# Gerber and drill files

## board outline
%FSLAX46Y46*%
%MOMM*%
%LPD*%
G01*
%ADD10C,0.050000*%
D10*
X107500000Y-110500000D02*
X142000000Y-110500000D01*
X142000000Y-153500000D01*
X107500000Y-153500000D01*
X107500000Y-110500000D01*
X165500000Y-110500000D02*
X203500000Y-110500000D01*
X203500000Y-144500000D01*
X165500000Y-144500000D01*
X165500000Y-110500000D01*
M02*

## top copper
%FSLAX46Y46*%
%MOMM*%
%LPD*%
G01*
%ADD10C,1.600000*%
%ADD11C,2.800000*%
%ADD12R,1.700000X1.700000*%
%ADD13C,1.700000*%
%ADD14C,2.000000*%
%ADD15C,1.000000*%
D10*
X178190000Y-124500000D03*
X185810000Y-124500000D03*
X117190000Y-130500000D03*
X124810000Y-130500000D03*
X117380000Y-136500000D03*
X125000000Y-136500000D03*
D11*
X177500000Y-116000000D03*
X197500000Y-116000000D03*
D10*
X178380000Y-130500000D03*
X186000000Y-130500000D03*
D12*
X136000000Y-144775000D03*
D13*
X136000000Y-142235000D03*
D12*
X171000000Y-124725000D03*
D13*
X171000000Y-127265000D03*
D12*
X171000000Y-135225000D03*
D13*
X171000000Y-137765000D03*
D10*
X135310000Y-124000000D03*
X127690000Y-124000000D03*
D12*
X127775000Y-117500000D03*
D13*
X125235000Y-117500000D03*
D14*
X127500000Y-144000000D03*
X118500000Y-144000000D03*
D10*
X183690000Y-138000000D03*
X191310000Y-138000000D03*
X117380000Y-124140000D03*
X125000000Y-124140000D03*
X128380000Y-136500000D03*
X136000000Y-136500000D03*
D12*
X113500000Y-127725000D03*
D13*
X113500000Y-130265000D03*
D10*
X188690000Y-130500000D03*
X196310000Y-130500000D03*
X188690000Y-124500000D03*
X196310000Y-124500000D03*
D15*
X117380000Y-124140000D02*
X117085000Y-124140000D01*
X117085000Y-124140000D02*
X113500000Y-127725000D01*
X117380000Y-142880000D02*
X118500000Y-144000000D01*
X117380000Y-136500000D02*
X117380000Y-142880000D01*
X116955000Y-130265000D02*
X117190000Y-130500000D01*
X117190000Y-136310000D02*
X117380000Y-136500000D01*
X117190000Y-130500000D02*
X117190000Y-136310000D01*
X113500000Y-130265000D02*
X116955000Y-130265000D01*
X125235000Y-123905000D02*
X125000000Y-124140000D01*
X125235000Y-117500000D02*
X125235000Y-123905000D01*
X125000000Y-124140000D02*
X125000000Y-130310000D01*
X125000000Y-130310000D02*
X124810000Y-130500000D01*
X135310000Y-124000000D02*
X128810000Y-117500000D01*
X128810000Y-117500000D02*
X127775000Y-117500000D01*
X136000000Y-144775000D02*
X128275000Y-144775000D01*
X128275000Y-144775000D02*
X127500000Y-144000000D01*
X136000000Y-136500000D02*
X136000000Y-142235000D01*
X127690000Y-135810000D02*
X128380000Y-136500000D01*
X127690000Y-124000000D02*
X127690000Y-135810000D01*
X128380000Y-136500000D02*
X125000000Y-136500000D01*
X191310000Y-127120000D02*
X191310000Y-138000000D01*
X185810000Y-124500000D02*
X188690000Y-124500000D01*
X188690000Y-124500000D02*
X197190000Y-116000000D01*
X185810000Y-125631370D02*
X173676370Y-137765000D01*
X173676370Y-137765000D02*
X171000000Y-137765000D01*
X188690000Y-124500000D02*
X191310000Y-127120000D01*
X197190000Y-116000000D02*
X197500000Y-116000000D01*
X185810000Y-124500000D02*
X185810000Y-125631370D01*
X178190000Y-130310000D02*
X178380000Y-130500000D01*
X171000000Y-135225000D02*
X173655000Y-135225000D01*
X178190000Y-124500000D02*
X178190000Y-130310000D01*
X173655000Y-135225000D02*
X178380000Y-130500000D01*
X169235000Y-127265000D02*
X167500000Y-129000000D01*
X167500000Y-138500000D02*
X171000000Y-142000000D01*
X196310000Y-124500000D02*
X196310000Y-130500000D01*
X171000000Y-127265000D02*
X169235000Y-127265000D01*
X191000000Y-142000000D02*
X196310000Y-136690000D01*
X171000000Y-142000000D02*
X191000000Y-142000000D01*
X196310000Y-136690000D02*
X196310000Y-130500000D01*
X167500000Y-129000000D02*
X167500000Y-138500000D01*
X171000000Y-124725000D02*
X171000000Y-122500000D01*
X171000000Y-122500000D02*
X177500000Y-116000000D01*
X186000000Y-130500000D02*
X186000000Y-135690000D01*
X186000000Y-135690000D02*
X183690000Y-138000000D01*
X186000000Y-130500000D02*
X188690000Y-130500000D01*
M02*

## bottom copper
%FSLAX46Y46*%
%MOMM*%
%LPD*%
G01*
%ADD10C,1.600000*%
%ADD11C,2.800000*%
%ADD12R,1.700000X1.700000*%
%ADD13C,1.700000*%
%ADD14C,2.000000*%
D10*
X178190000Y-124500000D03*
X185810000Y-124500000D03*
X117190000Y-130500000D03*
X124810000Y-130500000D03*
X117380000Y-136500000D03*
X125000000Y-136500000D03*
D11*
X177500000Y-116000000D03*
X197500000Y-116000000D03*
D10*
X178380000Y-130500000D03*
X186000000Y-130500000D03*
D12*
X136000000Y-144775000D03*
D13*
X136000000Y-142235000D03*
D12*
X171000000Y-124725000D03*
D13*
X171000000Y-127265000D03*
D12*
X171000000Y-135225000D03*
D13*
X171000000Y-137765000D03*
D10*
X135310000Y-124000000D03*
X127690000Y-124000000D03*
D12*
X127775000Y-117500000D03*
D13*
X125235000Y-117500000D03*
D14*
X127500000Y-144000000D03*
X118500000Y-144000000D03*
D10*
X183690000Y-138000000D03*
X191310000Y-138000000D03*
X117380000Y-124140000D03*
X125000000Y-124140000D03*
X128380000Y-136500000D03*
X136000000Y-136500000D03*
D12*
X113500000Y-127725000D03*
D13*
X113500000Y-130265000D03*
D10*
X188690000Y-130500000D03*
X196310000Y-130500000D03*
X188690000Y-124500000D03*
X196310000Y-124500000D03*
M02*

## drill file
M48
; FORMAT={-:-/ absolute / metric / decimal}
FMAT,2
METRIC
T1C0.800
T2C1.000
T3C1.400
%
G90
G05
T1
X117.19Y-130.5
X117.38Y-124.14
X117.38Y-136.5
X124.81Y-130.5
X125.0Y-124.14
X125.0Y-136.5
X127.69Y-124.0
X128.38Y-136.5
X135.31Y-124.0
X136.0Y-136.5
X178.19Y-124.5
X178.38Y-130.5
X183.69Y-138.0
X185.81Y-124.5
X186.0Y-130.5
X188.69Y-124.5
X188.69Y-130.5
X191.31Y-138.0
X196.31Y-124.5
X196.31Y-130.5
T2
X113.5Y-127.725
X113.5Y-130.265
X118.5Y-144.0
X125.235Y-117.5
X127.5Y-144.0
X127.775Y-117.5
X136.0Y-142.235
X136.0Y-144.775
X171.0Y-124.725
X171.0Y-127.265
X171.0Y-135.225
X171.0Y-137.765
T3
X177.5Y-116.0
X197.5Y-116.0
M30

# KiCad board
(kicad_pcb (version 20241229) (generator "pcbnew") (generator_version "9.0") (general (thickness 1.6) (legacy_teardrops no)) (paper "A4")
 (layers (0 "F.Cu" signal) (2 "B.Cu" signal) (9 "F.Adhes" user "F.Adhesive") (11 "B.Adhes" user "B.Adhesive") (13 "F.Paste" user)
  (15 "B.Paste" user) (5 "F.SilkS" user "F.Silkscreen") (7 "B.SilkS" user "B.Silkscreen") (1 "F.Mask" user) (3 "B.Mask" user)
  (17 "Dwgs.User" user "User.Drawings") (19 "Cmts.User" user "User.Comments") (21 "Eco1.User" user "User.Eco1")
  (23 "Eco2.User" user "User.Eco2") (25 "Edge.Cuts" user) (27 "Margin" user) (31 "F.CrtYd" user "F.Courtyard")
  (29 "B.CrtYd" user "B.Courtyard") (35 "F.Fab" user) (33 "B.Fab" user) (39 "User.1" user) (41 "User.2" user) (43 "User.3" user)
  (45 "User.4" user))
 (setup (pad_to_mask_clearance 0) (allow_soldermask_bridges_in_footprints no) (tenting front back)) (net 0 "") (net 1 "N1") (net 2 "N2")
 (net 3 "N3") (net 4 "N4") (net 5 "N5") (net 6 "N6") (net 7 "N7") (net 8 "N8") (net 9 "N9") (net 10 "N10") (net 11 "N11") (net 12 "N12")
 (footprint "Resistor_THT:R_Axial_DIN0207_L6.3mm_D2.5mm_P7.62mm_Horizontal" (layer "F.Cu") (at 178.19 124.5)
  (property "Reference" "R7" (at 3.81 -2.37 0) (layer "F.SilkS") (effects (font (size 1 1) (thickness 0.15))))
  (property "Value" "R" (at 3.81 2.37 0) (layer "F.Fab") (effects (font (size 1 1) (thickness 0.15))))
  (pad "1" thru_hole circle (at 0 0) (size 1.6 1.6) (drill 0.8) (layers "*.Cu" "*.Mask") (remove_unused_layers no) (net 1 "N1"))
  (pad "2" thru_hole circle (at 7.62 0) (size 1.6 1.6) (drill 0.8) (layers "*.Cu" "*.Mask") (remove_unused_layers no) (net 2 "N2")))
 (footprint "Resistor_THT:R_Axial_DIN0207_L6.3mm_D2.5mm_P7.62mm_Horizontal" (layer "F.Cu") (at 117.19 130.5)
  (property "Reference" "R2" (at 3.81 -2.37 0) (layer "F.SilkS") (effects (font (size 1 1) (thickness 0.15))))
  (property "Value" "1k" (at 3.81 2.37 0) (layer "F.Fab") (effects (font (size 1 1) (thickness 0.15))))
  (pad "1" thru_hole circle (at 0 0) (size 1.6 1.6) (drill 0.8) (layers "*.Cu" "*.Mask") (remove_unused_layers no) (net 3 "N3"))
  (pad "2" thru_hole circle (at 7.62 0) (size 1.6 1.6) (drill 0.8) (layers "*.Cu" "*.Mask") (remove_unused_layers no) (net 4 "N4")))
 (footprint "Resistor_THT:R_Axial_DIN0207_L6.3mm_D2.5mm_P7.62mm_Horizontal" (layer "F.Cu") (at 117.38 136.5)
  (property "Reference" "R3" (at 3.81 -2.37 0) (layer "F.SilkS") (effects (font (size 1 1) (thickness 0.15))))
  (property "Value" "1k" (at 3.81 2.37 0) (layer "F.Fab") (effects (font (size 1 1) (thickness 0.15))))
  (pad "1" thru_hole circle (at 0 0) (size 1.6 1.6) (drill 0.8) (layers "*.Cu" "*.Mask") (remove_unused_layers no) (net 3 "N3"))
  (pad "2" thru_hole circle (at 7.62 0) (size 1.6 1.6) (drill 0.8) (layers "*.Cu" "*.Mask") (remove_unused_layers no) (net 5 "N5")))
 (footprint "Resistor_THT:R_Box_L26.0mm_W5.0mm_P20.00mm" (layer "F.Cu") (at 177.5 116)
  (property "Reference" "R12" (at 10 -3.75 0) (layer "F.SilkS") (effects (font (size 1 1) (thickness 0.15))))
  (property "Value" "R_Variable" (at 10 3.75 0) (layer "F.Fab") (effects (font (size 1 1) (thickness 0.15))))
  (pad "1" thru_hole circle (at 0 0) (size 2.8 2.8) (drill 1.4) (layers "*.Cu" "*.Mask") (remove_unused_layers no) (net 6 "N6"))
  (pad "2" thru_hole circle (at 20 0) (size 2.8 2.8) (drill 1.4) (layers "*.Cu" "*.Mask") (remove_unused_layers no) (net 2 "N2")))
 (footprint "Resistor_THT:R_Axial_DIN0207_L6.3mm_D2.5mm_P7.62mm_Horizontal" (layer "F.Cu") (at 178.38 130.5)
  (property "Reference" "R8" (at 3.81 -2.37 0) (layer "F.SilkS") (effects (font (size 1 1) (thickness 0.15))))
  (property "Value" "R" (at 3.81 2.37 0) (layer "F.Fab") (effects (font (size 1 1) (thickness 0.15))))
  (pad "1" thru_hole circle (at 0 0) (size 1.6 1.6) (drill 0.8) (layers "*.Cu" "*.Mask") (remove_unused_layers no) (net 1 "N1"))
  (pad "2" thru_hole circle (at 7.62 0) (size 1.6 1.6) (drill 0.8) (layers "*.Cu" "*.Mask") (remove_unused_layers no) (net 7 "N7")))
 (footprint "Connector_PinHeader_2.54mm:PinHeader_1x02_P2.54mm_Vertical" (layer "F.Cu") (at 136 144.775 180)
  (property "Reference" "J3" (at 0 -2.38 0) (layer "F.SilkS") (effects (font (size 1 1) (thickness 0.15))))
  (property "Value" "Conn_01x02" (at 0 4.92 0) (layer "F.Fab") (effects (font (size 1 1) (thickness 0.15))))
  (pad "1" thru_hole rect (at 0 0 180) (size 1.7 1.7) (drill 1) (layers "*.Cu" "*.Mask") (remove_unused_layers no) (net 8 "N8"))
  (pad "2" thru_hole circle (at 0 2.54 180) (size 1.7 1.7) (drill 1) (layers "*.Cu" "*.Mask") (remove_unused_layers no) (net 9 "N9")))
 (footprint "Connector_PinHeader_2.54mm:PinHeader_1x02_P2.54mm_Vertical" (layer "F.Cu") (at 171 124.725)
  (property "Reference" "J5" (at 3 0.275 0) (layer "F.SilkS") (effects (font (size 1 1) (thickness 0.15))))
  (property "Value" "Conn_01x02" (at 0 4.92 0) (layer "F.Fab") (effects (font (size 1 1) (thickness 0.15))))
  (pad "1" thru_hole rect (at 0 0) (size 1.7 1.7) (drill 1) (layers "*.Cu" "*.Mask") (remove_unused_layers no) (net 6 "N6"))
  (pad "2" thru_hole circle (at 0 2.54) (size 1.7 1.7) (drill 1) (layers "*.Cu" "*.Mask") (remove_unused_layers no) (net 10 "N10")))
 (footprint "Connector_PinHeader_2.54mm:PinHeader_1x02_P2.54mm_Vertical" (layer "F.Cu") (at 171 135.225)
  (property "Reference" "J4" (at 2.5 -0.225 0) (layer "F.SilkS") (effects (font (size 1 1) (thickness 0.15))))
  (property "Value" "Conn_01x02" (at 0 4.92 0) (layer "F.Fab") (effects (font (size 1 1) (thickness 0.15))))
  (pad "1" thru_hole rect (at 0 0) (size 1.7 1.7) (drill 1) (layers "*.Cu" "*.Mask") (remove_unused_layers no) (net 1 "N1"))
  (pad "2" thru_hole circle (at 0 2.54) (size 1.7 1.7) (drill 1) (layers "*.Cu" "*.Mask") (remove_unused_layers no) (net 2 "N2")))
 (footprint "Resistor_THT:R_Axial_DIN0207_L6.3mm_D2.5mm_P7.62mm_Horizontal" (layer "F.Cu") (at 135.31 124 180)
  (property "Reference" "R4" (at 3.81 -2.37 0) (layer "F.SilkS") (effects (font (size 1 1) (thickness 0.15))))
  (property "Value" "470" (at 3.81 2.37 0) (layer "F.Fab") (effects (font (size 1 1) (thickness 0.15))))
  (pad "1" thru_hole circle (at 0 0 180) (size 1.6 1.6) (drill 0.8) (layers "*.Cu" "*.Mask") (remove_unused_layers no) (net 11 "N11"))
  (pad "2" thru_hole circle (at 7.62 0 180) (size 1.6 1.6) (drill 0.8) (layers "*.Cu" "*.Mask") (remove_unused_layers no) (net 5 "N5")))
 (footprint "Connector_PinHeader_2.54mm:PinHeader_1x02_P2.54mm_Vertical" (layer "F.Cu") (at 127.775 117.5 -90)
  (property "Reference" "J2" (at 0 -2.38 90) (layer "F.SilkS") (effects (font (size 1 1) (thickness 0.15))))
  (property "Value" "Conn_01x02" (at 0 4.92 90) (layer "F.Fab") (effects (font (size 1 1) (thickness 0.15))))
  (pad "1" thru_hole rect (at 0 0 270) (size 1.7 1.7) (drill 1) (layers "*.Cu" "*.Mask") (remove_unused_layers no) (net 11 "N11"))
  (pad "2" thru_hole circle (at 0 2.54 270) (size 1.7 1.7) (drill 1) (layers "*.Cu" "*.Mask") (remove_unused_layers no) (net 4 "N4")))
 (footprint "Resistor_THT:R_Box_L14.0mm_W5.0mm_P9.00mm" (layer "F.Cu") (at 127.5 144 180)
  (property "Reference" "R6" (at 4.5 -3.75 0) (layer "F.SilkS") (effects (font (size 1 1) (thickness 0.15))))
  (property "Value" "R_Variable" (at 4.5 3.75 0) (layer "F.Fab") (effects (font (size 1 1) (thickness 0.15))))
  (pad "1" thru_hole circle (at 0 0 180) (size 2 2) (drill 1) (layers "*.Cu" "*.Mask") (remove_unused_layers no) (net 8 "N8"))
  (pad "2" thru_hole circle (at 9 0 180) (size 2 2) (drill 1) (layers "*.Cu" "*.Mask") (remove_unused_layers no) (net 3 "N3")))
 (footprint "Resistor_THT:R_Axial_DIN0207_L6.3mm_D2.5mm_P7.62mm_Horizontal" (layer "F.Cu") (at 183.69 138)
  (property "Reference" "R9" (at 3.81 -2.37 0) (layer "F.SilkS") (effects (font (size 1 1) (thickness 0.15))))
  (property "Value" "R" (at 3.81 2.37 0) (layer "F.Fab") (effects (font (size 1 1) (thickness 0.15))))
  (pad "1" thru_hole circle (at 0 0) (size 1.6 1.6) (drill 0.8) (layers "*.Cu" "*.Mask") (remove_unused_layers no) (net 7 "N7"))
  (pad "2" thru_hole circle (at 7.62 0) (size 1.6 1.6) (drill 0.8) (layers "*.Cu" "*.Mask") (remove_unused_layers no) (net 2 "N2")))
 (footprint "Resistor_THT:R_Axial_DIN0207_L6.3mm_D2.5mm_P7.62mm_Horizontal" (layer "F.Cu") (at 117.38 124.14)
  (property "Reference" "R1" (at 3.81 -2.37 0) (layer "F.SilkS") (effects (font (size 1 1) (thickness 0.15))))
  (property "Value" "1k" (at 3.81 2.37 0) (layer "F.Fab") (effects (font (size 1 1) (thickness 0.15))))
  (pad "1" thru_hole circle (at 0 0) (size 1.6 1.6) (drill 0.8) (layers "*.Cu" "*.Mask") (remove_unused_layers no) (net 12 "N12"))
  (pad "2" thru_hole circle (at 7.62 0) (size 1.6 1.6) (drill 0.8) (layers "*.Cu" "*.Mask") (remove_unused_layers no) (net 4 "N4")))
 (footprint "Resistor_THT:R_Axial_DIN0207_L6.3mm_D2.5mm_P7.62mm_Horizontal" (layer "F.Cu") (at 128.38 136.5)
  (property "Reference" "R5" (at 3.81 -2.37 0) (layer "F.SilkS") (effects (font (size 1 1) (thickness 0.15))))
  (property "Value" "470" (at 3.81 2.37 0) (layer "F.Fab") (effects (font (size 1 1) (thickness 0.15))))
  (pad "1" thru_hole circle (at 0 0) (size 1.6 1.6) (drill 0.8) (layers "*.Cu" "*.Mask") (remove_unused_layers no) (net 5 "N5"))
  (pad "2" thru_hole circle (at 7.62 0) (size 1.6 1.6) (drill 0.8) (layers "*.Cu" "*.Mask") (remove_unused_layers no) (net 9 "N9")))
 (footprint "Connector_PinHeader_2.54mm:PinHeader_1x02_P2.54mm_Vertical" (layer "F.Cu") (at 113.5 127.725)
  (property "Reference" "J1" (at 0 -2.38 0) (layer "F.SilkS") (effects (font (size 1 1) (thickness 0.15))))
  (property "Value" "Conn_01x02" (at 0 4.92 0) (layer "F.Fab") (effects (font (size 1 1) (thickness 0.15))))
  (pad "1" thru_hole rect (at 0 0) (size 1.7 1.7) (drill 1) (layers "*.Cu" "*.Mask") (remove_unused_layers no) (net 12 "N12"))
  (pad "2" thru_hole circle (at 0 2.54) (size 1.7 1.7) (drill 1) (layers "*.Cu" "*.Mask") (remove_unused_layers no) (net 3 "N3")))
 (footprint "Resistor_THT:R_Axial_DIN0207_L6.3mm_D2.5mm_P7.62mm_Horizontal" (layer "F.Cu") (at 188.69 130.5)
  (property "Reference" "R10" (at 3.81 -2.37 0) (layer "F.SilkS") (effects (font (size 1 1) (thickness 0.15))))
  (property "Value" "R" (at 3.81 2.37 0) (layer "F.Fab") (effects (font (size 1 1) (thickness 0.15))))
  (pad "1" thru_hole circle (at 0 0) (size 1.6 1.6) (drill 0.8) (layers "*.Cu" "*.Mask") (remove_unused_layers no) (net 7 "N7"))
  (pad "2" thru_hole circle (at 7.62 0) (size 1.6 1.6) (drill 0.8) (layers "*.Cu" "*.Mask") (remove_unused_layers no) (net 10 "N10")))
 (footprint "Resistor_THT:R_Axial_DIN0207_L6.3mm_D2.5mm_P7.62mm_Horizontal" (layer "F.Cu") (at 188.69 124.5)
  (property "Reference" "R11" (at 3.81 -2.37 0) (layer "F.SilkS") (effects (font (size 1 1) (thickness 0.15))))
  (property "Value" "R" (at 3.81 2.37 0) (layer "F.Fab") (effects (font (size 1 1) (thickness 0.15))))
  (pad "1" thru_hole circle (at 0 0) (size 1.6 1.6) (drill 0.8) (layers "*.Cu" "*.Mask") (remove_unused_layers no) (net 2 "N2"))
  (pad "2" thru_hole circle (at 7.62 0) (size 1.6 1.6) (drill 0.8) (layers "*.Cu" "*.Mask") (remove_unused_layers no) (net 10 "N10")))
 (gr_rect (start 107.5 110.5) (end 142 153.5) (stroke (width 0.05) (type default)) (fill no) (layer "Edge.Cuts"))
 (gr_rect (start 165.5 110.5) (end 203.5 144.5) (stroke (width 0.05) (type default)) (fill no) (layer "Edge.Cuts"))
 (segment (start 117.38 124.14) (end 117.085 124.14) (width 1) (layer "F.Cu") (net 12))
 (segment (start 117.085 124.14) (end 113.5 127.725) (width 1) (layer "F.Cu") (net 12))
 (segment (start 117.38 142.88) (end 118.5 144) (width 1) (layer "F.Cu") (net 3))
 (segment (start 117.38 136.5) (end 117.38 142.88) (width 1) (layer "F.Cu") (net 3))
 (segment (start 116.955 130.265) (end 117.19 130.5) (width 1) (layer "F.Cu") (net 3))
 (segment (start 117.19 136.31) (end 117.38 136.5) (width 1) (layer "F.Cu") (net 3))
 (segment (start 117.19 130.5) (end 117.19 136.31) (width 1) (layer "F.Cu") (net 3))
 (segment (start 113.5 130.265) (end 116.955 130.265) (width 1) (layer "F.Cu") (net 3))
 (segment (start 125.235 123.905) (end 125 124.14) (width 1) (layer "F.Cu") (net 4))
 (segment (start 125.235 117.5) (end 125.235 123.905) (width 1) (layer "F.Cu") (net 4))
 (segment (start 125 124.14) (end 125 130.31) (width 1) (layer "F.Cu") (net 4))
 (segment (start 125 130.31) (end 124.81 130.5) (width 1) (layer "F.Cu") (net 4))
 (segment (start 135.31 124) (end 128.81 117.5) (width 1) (layer "F.Cu") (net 11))
 (segment (start 128.81 117.5) (end 127.775 117.5) (width 1) (layer "F.Cu") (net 11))
 (segment (start 136 144.775) (end 128.275 144.775) (width 1) (layer "F.Cu") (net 8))
 (segment (start 128.275 144.775) (end 127.5 144) (width 1) (layer "F.Cu") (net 8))
 (segment (start 136 136.5) (end 136 142.235) (width 1) (layer "F.Cu") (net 9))
 (segment (start 127.69 135.81) (end 128.38 136.5) (width 1) (layer "F.Cu") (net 5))
 (segment (start 127.69 124) (end 127.69 135.81) (width 1) (layer "F.Cu") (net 5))
 (segment (start 128.38 136.5) (end 125 136.5) (width 1) (layer "F.Cu") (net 5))
 (segment (start 191.31 127.12) (end 191.31 138) (width 1) (layer "F.Cu") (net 2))
 (segment (start 185.81 124.5) (end 188.69 124.5) (width 1) (layer "F.Cu") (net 2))
 (segment (start 188.69 124.5) (end 197.19 116) (width 1) (layer "F.Cu") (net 2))
 (segment (start 185.81 125.63137) (end 173.67637 137.765) (width 1) (layer "F.Cu") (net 2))
 (segment (start 173.67637 137.765) (end 171 137.765) (width 1) (layer "F.Cu") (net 2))
 (segment (start 188.69 124.5) (end 191.31 127.12) (width 1) (layer "F.Cu") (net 2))
 (segment (start 197.19 116) (end 197.5 116) (width 1) (layer "F.Cu") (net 2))
 (segment (start 185.81 124.5) (end 185.81 125.63137) (width 1) (layer "F.Cu") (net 2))
 (segment (start 178.19 130.31) (end 178.38 130.5) (width 1) (layer "F.Cu") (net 1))
 (segment (start 171 135.225) (end 173.655 135.225) (width 1) (layer "F.Cu") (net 1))
 (segment (start 178.19 124.5) (end 178.19 130.31) (width 1) (layer "F.Cu") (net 1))
 (segment (start 173.655 135.225) (end 178.38 130.5) (width 1) (layer "F.Cu") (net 1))
 (segment (start 169.235 127.265) (end 167.5 129) (width 1) (layer "F.Cu") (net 10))
 (segment (start 167.5 138.5) (end 171 142) (width 1) (layer "F.Cu") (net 10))
 (segment (start 196.31 124.5) (end 196.31 130.5) (width 1) (layer "F.Cu") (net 10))
 (segment (start 171 127.265) (end 169.235 127.265) (width 1) (layer "F.Cu") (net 10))
 (segment (start 191 142) (end 196.31 136.69) (width 1) (layer "F.Cu") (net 10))
 (segment (start 171 142) (end 191 142) (width 1) (layer "F.Cu") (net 10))
 (segment (start 196.31 136.69) (end 196.31 130.5) (width 1) (layer "F.Cu") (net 10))
 (segment (start 167.5 129) (end 167.5 138.5) (width 1) (layer "F.Cu") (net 10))
 (segment (start 171 124.725) (end 171 122.5) (width 1) (layer "F.Cu") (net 6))
 (segment (start 171 122.5) (end 177.5 116) (width 1) (layer "F.Cu") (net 6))
 (segment (start 186 130.5) (end 186 135.69) (width 1) (layer "F.Cu") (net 7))
 (segment (start 186 135.69) (end 183.69 138) (width 1) (layer "F.Cu") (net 7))
 (segment (start 186 130.5) (end 188.69 130.5) (width 1) (layer "F.Cu") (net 7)))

